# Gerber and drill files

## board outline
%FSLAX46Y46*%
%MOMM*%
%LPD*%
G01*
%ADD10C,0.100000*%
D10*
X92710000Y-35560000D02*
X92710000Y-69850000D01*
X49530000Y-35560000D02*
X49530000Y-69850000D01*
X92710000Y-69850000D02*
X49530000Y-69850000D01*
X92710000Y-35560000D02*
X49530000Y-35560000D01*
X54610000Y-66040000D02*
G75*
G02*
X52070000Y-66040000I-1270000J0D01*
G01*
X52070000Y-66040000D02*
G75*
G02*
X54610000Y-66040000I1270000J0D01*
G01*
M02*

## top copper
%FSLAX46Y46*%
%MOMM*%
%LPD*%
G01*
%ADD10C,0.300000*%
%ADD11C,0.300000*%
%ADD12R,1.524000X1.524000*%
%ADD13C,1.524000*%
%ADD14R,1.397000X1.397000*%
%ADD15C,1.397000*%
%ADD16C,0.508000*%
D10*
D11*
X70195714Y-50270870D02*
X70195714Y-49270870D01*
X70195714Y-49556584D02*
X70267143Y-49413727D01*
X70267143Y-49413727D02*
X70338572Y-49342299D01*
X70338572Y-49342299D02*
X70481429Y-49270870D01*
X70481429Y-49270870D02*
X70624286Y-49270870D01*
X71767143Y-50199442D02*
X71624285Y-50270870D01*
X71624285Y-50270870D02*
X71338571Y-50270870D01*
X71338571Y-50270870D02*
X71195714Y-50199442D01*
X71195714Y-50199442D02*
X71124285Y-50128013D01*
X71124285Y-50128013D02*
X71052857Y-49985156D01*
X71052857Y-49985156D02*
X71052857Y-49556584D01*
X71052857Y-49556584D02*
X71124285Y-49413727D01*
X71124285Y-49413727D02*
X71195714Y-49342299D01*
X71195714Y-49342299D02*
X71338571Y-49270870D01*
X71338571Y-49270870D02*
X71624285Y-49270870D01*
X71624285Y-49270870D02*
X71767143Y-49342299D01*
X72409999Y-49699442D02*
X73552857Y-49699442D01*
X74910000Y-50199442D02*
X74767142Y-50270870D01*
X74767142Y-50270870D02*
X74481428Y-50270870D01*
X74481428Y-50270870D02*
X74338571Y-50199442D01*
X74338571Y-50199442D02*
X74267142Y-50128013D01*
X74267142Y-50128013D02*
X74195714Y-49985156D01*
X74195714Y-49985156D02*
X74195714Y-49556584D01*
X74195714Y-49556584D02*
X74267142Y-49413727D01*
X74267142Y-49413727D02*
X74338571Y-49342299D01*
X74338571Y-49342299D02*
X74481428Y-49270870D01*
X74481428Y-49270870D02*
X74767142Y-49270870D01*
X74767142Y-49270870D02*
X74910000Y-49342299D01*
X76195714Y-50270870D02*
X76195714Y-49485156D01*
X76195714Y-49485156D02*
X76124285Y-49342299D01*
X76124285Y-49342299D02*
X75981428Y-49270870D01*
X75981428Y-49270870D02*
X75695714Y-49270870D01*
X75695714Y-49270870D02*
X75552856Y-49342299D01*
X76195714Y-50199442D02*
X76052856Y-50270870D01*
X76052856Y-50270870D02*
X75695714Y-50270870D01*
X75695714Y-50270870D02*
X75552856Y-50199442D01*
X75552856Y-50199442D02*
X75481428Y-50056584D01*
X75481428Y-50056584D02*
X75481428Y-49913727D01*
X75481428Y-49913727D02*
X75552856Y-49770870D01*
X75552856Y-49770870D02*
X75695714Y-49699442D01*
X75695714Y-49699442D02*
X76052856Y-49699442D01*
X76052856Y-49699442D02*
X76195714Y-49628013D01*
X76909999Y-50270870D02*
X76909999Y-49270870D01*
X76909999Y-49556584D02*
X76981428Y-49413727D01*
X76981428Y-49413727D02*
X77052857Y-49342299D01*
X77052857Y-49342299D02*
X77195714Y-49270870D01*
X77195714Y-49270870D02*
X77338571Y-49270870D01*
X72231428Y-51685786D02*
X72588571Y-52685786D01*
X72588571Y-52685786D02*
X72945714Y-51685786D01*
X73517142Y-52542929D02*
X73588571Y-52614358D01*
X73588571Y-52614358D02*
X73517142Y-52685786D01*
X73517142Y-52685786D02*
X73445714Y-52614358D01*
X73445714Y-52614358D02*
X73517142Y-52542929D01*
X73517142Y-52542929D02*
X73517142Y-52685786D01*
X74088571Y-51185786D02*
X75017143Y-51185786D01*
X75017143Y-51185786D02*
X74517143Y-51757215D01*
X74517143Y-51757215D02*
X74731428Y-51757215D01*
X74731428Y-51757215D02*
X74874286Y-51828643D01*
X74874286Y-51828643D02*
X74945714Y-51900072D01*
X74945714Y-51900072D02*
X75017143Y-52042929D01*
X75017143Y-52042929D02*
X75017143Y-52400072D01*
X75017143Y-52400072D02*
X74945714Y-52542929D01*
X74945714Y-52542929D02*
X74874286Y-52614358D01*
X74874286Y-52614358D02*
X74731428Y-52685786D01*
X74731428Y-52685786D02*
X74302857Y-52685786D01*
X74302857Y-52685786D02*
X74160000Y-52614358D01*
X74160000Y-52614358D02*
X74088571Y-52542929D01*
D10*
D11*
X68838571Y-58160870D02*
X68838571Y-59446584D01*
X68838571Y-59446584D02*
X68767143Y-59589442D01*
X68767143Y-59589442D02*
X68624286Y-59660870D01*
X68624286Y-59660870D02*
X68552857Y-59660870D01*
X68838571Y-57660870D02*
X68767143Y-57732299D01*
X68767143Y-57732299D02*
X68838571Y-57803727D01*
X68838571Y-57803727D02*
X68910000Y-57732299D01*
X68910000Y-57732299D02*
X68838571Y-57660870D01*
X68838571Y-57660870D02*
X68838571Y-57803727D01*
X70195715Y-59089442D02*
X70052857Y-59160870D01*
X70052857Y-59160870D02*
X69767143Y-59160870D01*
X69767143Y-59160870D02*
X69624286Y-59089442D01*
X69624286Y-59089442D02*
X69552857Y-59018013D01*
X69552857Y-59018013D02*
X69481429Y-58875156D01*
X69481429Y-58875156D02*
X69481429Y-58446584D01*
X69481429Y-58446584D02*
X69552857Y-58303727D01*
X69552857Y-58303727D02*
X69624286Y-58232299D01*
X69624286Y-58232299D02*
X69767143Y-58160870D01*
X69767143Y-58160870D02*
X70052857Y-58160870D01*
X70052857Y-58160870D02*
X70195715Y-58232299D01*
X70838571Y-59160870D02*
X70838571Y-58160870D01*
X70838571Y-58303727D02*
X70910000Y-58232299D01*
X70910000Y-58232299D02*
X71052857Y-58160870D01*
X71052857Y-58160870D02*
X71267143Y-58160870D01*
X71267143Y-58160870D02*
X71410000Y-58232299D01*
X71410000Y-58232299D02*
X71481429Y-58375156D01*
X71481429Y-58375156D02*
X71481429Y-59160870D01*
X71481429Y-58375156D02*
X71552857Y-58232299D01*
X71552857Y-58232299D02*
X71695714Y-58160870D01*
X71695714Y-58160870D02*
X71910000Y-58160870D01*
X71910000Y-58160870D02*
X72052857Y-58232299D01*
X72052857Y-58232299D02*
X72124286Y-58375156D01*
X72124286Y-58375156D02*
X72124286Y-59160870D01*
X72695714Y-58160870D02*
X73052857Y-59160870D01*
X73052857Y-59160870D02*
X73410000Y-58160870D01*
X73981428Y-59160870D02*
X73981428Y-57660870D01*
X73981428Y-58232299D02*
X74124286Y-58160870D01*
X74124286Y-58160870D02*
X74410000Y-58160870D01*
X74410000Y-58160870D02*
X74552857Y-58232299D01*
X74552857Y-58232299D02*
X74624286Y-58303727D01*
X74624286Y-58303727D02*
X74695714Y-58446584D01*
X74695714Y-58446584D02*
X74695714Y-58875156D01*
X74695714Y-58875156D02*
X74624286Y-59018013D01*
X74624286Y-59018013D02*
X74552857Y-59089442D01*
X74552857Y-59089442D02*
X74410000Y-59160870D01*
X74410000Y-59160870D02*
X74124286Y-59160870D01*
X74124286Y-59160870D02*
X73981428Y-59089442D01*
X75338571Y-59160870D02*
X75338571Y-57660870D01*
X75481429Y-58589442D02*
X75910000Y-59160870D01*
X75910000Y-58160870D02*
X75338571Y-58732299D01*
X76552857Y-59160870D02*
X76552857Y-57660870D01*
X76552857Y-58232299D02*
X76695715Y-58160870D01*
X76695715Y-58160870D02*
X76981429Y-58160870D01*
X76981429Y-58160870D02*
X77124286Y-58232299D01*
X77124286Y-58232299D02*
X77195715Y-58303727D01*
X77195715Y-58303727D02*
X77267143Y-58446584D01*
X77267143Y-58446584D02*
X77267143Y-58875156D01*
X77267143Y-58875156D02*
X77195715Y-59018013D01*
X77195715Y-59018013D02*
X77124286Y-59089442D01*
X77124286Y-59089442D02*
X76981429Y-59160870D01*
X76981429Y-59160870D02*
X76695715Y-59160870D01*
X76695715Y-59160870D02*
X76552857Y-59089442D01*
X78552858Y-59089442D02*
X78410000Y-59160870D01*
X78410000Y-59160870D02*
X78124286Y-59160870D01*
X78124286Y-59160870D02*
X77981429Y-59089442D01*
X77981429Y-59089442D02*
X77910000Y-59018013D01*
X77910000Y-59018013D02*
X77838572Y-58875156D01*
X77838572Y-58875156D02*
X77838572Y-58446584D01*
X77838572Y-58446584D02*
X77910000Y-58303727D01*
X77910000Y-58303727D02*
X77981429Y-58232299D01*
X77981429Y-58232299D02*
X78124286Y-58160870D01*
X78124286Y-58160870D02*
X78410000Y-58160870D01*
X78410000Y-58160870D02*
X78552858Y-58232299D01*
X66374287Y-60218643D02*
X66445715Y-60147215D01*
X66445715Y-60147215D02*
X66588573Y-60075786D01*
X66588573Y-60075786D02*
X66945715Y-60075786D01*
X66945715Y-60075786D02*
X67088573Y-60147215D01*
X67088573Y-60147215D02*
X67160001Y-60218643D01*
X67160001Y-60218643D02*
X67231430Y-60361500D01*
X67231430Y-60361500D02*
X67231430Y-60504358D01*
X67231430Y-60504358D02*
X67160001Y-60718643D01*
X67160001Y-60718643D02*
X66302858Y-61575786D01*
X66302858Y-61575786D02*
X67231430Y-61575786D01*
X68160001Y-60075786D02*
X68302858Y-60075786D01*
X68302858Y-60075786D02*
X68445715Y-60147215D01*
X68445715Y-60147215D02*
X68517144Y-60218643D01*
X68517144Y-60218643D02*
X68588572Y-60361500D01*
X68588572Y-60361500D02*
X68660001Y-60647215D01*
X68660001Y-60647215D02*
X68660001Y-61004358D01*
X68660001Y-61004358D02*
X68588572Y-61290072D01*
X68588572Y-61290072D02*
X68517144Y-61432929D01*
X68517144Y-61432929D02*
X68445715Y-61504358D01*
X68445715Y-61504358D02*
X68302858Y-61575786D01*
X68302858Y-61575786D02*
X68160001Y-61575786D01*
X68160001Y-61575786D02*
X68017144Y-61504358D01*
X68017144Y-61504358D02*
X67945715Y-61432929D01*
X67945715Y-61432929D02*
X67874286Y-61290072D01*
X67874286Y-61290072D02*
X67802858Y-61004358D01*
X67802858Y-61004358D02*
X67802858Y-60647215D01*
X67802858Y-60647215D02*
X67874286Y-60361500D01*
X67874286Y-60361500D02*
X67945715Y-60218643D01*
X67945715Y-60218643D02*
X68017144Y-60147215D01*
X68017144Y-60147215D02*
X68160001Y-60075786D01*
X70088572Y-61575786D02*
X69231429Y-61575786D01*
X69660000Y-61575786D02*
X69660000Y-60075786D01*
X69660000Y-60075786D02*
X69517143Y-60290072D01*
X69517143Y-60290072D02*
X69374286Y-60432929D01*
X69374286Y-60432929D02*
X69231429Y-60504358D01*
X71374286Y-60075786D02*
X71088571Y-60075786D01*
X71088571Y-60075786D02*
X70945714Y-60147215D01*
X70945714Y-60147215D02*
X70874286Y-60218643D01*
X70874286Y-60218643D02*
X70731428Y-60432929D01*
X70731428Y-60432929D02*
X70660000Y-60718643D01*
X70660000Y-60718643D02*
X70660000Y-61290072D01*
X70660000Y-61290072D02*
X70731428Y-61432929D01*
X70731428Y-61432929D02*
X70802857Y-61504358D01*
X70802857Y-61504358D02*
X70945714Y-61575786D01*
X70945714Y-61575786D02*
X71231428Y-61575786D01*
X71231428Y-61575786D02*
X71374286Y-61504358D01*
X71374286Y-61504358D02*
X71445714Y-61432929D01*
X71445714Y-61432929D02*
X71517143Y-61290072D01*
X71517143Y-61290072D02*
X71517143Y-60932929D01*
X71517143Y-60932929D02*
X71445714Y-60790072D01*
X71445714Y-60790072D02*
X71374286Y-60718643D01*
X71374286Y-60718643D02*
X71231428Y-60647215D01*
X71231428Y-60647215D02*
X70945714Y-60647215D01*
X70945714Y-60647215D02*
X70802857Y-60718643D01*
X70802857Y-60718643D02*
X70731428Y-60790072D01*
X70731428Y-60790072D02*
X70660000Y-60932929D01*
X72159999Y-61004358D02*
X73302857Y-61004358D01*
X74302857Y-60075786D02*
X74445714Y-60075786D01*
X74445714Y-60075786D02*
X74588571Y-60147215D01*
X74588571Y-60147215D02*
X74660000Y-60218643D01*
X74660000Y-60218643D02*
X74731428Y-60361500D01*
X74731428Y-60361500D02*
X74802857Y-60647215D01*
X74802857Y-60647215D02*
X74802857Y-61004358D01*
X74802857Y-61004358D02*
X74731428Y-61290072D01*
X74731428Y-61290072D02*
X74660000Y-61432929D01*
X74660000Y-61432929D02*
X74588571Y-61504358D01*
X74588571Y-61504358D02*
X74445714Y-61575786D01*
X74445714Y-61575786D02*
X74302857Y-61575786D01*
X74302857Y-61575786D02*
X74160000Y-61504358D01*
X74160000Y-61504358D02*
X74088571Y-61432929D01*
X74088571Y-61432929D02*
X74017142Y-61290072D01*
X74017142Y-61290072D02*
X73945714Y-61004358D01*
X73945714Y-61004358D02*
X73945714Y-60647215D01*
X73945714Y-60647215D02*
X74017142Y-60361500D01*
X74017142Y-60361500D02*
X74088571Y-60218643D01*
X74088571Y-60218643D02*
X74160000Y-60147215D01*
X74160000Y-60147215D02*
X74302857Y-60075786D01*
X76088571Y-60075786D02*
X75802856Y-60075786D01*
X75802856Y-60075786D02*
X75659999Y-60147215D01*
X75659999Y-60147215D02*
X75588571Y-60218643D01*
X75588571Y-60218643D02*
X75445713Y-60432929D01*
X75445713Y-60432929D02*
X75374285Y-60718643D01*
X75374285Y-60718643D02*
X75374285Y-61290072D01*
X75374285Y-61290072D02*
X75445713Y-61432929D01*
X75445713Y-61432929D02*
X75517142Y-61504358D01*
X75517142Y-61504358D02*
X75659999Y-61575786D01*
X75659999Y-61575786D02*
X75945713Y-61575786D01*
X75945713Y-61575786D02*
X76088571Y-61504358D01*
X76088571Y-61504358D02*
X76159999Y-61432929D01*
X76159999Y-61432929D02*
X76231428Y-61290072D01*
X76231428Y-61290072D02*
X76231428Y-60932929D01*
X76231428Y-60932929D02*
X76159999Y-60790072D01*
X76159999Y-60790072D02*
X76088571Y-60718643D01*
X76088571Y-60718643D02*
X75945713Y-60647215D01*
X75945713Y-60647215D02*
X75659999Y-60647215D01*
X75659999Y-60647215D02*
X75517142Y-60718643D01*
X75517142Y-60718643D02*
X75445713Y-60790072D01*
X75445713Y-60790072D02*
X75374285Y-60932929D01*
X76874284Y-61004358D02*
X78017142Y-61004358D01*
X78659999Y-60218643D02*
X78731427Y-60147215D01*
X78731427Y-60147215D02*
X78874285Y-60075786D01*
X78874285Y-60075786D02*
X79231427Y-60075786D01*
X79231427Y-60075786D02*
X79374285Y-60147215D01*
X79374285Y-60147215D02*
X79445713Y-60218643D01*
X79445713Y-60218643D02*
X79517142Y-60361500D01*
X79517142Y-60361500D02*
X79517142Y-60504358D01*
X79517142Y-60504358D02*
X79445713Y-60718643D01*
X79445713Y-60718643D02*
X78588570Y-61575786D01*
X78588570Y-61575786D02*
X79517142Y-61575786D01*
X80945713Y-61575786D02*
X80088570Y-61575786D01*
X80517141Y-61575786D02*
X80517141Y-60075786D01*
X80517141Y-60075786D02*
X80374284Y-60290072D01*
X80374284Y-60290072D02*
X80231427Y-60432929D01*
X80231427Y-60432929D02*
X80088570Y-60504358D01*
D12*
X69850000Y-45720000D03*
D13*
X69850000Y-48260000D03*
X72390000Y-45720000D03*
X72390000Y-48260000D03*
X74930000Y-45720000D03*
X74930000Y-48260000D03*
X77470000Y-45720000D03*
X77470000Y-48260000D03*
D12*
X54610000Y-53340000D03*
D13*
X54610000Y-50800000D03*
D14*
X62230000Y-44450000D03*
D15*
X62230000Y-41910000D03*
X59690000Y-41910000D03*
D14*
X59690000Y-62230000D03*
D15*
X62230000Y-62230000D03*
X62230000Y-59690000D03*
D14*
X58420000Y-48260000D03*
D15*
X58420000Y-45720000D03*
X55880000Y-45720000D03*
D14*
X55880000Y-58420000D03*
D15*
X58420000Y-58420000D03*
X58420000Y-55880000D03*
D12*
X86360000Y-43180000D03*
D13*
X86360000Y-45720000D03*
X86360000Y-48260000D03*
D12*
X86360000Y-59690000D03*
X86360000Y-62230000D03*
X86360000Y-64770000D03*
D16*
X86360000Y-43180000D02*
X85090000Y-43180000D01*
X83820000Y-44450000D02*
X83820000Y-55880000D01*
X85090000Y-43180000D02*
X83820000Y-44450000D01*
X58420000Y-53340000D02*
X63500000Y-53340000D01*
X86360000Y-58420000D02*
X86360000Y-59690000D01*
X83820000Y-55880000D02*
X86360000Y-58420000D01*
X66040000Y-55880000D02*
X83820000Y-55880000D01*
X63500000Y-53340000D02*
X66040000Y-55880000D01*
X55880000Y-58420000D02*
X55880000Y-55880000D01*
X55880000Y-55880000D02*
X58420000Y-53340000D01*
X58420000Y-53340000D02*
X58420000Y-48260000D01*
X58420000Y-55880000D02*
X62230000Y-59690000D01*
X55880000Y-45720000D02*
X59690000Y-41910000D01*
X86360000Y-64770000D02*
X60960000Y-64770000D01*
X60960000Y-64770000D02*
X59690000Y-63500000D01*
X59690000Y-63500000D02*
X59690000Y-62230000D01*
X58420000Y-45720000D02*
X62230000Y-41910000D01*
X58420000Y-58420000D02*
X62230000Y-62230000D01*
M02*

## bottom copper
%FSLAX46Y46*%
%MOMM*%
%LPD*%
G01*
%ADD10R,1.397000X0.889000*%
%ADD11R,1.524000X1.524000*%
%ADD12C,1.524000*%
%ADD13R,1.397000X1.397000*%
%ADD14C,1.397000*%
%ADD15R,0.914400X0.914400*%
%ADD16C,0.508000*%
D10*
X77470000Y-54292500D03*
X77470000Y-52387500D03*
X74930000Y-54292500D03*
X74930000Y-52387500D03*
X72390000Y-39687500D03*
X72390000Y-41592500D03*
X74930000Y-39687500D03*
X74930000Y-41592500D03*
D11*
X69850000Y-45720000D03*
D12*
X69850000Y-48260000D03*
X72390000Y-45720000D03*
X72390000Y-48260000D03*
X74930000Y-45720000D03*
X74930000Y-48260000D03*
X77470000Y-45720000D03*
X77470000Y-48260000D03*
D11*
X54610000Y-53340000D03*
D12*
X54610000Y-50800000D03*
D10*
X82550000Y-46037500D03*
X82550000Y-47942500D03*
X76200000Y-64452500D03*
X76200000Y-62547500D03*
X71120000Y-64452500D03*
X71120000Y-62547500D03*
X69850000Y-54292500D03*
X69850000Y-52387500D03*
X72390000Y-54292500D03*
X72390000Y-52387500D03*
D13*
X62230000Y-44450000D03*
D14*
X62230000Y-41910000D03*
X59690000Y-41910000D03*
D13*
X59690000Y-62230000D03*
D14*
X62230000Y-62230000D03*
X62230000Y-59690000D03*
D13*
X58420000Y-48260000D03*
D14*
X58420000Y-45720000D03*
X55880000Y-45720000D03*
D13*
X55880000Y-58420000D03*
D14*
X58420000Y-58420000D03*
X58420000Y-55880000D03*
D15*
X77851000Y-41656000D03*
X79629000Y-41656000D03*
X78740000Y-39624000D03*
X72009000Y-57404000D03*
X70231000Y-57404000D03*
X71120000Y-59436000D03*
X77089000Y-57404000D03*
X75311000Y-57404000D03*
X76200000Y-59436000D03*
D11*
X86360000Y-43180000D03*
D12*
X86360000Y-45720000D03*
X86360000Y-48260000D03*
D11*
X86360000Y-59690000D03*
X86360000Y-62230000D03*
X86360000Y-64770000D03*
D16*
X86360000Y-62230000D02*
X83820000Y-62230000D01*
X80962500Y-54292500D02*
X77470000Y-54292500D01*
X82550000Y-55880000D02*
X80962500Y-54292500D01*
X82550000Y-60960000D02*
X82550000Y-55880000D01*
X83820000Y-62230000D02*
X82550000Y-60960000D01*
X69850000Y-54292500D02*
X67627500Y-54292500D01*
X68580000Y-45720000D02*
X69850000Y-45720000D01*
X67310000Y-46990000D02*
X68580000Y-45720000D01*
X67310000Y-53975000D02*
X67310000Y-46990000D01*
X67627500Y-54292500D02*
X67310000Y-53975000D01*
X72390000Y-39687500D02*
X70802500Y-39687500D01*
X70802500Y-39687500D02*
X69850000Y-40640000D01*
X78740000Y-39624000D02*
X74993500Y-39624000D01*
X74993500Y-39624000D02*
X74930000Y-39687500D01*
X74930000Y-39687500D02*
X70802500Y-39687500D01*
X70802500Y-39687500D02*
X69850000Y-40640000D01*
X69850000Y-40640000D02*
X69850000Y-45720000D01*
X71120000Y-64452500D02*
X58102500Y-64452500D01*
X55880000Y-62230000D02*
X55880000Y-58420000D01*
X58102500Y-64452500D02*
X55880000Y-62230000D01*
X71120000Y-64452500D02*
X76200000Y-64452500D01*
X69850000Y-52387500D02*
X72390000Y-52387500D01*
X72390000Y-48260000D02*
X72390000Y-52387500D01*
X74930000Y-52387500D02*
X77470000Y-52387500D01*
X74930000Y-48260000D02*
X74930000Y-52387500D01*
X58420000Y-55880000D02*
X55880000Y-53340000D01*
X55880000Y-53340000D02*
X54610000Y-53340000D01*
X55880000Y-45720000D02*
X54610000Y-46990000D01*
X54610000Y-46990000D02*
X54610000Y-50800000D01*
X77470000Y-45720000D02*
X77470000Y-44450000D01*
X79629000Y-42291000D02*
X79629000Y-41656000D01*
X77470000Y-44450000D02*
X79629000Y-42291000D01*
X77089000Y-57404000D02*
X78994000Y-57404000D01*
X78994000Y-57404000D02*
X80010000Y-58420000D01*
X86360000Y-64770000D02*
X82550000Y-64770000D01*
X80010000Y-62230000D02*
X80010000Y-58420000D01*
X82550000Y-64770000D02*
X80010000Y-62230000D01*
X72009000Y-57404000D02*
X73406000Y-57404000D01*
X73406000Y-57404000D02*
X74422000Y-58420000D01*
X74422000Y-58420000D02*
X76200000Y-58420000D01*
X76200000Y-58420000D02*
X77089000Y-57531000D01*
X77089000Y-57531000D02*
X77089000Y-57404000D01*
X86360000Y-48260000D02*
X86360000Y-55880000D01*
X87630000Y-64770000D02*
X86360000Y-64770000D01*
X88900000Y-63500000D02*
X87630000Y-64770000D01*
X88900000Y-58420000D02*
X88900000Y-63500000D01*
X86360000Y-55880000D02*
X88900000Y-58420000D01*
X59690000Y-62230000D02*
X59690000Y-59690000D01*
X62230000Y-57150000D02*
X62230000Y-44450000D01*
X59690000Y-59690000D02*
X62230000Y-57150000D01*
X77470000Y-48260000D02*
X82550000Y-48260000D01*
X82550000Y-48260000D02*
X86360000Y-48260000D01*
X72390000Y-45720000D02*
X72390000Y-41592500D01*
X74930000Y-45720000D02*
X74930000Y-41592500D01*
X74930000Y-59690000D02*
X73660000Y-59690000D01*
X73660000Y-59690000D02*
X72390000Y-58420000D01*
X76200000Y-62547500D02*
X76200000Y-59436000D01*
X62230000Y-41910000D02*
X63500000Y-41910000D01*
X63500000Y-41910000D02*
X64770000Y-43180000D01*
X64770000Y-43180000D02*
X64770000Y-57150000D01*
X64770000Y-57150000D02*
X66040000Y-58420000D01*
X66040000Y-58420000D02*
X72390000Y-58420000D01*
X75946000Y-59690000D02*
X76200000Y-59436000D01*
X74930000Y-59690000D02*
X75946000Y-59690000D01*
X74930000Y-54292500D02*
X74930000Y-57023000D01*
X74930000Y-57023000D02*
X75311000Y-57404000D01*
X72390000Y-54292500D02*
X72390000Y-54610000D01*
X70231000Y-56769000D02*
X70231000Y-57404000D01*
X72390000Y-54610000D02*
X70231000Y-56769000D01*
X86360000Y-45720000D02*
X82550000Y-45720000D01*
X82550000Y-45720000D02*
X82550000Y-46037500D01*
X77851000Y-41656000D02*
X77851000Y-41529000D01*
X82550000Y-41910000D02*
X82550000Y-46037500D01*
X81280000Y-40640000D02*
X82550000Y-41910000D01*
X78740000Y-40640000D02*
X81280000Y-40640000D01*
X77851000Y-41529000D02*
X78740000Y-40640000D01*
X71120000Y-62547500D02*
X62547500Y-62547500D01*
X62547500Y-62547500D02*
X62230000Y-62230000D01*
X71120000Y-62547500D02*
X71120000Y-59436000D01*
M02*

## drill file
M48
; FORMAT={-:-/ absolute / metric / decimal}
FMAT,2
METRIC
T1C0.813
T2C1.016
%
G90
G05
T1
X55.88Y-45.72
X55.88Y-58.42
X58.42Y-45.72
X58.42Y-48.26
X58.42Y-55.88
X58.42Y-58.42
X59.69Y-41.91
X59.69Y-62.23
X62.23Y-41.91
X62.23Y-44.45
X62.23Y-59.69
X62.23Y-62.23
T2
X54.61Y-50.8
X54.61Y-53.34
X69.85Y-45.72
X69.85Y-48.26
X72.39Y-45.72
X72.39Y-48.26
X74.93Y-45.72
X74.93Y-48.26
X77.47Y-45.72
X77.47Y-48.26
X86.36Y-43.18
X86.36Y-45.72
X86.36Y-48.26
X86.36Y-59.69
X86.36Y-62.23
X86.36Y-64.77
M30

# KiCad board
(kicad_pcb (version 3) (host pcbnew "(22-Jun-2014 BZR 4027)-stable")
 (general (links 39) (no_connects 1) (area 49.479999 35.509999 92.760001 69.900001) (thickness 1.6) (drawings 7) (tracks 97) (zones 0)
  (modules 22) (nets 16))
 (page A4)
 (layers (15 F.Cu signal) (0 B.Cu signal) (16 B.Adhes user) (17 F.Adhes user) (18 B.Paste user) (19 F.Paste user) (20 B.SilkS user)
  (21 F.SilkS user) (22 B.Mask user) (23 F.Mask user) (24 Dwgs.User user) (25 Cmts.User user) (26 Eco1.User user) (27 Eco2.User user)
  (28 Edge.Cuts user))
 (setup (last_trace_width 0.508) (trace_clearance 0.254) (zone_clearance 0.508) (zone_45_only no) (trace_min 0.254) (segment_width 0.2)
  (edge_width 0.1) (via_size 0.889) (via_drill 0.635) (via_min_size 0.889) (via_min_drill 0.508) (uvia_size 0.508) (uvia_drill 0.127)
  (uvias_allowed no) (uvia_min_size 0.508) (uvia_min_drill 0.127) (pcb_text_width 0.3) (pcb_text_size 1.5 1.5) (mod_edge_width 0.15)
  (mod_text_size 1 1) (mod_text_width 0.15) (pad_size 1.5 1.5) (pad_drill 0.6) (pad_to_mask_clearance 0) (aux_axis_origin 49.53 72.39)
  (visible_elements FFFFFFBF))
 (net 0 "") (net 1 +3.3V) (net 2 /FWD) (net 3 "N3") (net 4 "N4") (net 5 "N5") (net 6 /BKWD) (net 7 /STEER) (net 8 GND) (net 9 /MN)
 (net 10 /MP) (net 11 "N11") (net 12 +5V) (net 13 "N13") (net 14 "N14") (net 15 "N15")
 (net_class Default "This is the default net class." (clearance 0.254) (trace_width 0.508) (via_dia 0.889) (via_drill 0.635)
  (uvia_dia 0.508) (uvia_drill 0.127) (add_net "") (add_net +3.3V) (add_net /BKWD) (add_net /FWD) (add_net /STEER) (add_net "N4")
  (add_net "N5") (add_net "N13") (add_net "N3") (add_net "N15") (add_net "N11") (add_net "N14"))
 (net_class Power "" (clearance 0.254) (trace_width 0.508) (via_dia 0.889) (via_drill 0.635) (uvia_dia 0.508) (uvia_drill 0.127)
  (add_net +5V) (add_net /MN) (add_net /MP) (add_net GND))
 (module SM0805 (layer B.Cu) (at 77.47 53.34 90)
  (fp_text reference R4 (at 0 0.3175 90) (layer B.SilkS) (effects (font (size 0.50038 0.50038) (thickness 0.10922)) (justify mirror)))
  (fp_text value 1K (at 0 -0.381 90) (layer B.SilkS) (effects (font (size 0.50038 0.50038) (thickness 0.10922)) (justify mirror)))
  (pad 1 smd rect (at -0.9525 0 90) (size 0.889 1.397) (layers B.Cu B.Paste B.Mask) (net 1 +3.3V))
  (pad 2 smd rect (at 0.9525 0 90) (size 0.889 1.397) (layers B.Cu B.Paste B.Mask) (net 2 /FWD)))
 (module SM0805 (layer B.Cu) (at 74.93 53.34 90)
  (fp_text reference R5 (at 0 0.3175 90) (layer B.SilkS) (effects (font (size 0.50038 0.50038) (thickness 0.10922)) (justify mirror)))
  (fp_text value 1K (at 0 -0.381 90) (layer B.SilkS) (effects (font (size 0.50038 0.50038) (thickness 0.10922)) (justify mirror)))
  (pad 1 smd rect (at -0.9525 0 90) (size 0.889 1.397) (layers B.Cu B.Paste B.Mask) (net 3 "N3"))
  (pad 2 smd rect (at 0.9525 0 90) (size 0.889 1.397) (layers B.Cu B.Paste B.Mask) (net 2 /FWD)))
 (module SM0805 (layer B.Cu) (at 72.39 40.64 270)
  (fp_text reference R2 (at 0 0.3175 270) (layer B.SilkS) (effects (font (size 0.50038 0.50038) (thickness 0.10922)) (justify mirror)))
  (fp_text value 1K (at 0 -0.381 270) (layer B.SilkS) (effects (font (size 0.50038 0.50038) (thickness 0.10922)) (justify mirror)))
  (pad 1 smd rect (at -0.9525 0 270) (size 0.889 1.397) (layers B.Cu B.Paste B.Mask) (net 1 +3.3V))
  (pad 2 smd rect (at 0.9525 0 270) (size 0.889 1.397) (layers B.Cu B.Paste B.Mask) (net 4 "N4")))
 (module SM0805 (layer B.Cu) (at 74.93 40.64 270)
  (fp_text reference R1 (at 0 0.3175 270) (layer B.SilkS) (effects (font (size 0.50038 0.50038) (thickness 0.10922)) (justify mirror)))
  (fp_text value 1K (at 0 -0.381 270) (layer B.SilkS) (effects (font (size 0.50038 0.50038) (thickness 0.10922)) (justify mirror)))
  (pad 1 smd rect (at -0.9525 0 270) (size 0.889 1.397) (layers B.Cu B.Paste B.Mask) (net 1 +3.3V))
  (pad 2 smd rect (at 0.9525 0 270) (size 0.889 1.397) (layers B.Cu B.Paste B.Mask) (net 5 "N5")))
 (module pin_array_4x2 (layer B.Cu) (at 73.66 46.99)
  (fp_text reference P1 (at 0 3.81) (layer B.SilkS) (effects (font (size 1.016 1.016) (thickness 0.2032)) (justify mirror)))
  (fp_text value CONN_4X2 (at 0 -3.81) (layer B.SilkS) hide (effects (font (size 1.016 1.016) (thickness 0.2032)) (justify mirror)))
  (pad 1 thru_hole rect (at -3.81 -1.27) (size 1.524 1.524) (drill 1.016) (layers *.Cu *.Mask B.SilkS) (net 1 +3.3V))
  (pad 2 thru_hole circle (at -3.81 1.27) (size 1.524 1.524) (drill 1.016) (layers *.Cu *.Mask B.SilkS))
  (pad 3 thru_hole circle (at -1.27 -1.27) (size 1.524 1.524) (drill 1.016) (layers *.Cu *.Mask B.SilkS) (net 4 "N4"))
  (pad 4 thru_hole circle (at -1.27 1.27) (size 1.524 1.524) (drill 1.016) (layers *.Cu *.Mask B.SilkS) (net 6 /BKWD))
  (pad 5 thru_hole circle (at 1.27 -1.27) (size 1.524 1.524) (drill 1.016) (layers *.Cu *.Mask B.SilkS) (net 5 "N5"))
  (pad 6 thru_hole circle (at 1.27 1.27) (size 1.524 1.524) (drill 1.016) (layers *.Cu *.Mask B.SilkS) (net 2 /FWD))
  (pad 7 thru_hole circle (at 3.81 -1.27) (size 1.524 1.524) (drill 1.016) (layers *.Cu *.Mask B.SilkS) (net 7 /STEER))
  (pad 8 thru_hole circle (at 3.81 1.27) (size 1.524 1.524) (drill 1.016) (layers *.Cu *.Mask B.SilkS) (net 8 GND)))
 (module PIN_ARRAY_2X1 (layer F.Cu) (at 54.61 52.07 90)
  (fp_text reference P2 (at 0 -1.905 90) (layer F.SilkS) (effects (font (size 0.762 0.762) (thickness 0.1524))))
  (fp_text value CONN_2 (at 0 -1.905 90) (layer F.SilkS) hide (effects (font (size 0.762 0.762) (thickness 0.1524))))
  (pad 1 thru_hole rect (at -1.27 0 90) (size 1.524 1.524) (drill 1.016) (layers *.Cu *.Mask F.SilkS) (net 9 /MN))
  (pad 2 thru_hole circle (at 1.27 0 90) (size 1.524 1.524) (drill 1.016) (layers *.Cu *.Mask F.SilkS) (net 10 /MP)))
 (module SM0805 (layer B.Cu) (at 82.55 46.99 270)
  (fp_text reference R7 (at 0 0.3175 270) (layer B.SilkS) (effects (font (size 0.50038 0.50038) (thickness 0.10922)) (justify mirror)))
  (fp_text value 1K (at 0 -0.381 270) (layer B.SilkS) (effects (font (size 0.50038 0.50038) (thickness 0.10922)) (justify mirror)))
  (pad 1 smd rect (at -0.9525 0 270) (size 0.889 1.397) (layers B.Cu B.Paste B.Mask) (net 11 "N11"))
  (pad 2 smd rect (at 0.9525 0 270) (size 0.889 1.397) (layers B.Cu B.Paste B.Mask) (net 8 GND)))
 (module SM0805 (layer B.Cu) (at 76.2 63.5 90)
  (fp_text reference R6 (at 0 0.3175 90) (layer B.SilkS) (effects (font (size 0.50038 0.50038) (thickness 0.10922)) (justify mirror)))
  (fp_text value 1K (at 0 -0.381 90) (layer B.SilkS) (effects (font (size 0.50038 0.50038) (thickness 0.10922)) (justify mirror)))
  (pad 1 smd rect (at -0.9525 0 90) (size 0.889 1.397) (layers B.Cu B.Paste B.Mask) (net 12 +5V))
  (pad 2 smd rect (at 0.9525 0 90) (size 0.889 1.397) (layers B.Cu B.Paste B.Mask) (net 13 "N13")))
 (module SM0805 (layer B.Cu) (at 71.12 63.5 90)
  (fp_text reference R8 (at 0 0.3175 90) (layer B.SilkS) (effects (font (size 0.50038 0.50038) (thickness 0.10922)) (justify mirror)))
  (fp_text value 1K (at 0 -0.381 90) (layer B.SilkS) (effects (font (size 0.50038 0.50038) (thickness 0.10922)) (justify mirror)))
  (pad 1 smd rect (at -0.9525 0 90) (size 0.889 1.397) (layers B.Cu B.Paste B.Mask) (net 12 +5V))
  (pad 2 smd rect (at 0.9525 0 90) (size 0.889 1.397) (layers B.Cu B.Paste B.Mask) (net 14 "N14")))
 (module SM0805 (layer B.Cu) (at 69.85 53.34 90)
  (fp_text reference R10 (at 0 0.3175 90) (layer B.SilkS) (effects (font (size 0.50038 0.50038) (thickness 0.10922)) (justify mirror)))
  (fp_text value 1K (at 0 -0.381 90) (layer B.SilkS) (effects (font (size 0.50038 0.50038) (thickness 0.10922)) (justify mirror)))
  (pad 1 smd rect (at -0.9525 0 90) (size 0.889 1.397) (layers B.Cu B.Paste B.Mask) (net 1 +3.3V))
  (pad 2 smd rect (at 0.9525 0 90) (size 0.889 1.397) (layers B.Cu B.Paste B.Mask) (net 6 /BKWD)))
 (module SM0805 (layer B.Cu) (at 72.39 53.34 90)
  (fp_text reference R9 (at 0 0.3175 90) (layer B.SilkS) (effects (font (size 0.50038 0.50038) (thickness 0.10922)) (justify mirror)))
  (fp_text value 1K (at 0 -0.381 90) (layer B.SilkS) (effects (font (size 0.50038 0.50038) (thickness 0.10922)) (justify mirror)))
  (pad 1 smd rect (at -0.9525 0 90) (size 0.889 1.397) (layers B.Cu B.Paste B.Mask) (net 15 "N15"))
  (pad 2 smd rect (at 0.9525 0 90) (size 0.889 1.397) (layers B.Cu B.Paste B.Mask) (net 6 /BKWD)))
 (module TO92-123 (layer F.Cu) (at 60.96 43.18 270)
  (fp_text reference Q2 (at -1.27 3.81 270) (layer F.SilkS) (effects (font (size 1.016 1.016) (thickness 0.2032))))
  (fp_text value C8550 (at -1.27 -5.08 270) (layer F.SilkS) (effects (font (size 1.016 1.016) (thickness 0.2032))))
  (pad 3 thru_hole rect (at 1.27 -1.27 270) (size 1.397 1.397) (drill 0.8128) (layers *.Cu *.Mask F.SilkS) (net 8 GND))
  (pad 2 thru_hole circle (at -1.27 -1.27 270) (size 1.397 1.397) (drill 0.8128) (layers *.Cu *.Mask F.SilkS) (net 13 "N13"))
  (pad 1 thru_hole circle (at -1.27 1.27 270) (size 1.397 1.397) (drill 0.8128) (layers *.Cu *.Mask F.SilkS) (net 10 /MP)))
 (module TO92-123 (layer F.Cu) (at 60.96 60.96 180)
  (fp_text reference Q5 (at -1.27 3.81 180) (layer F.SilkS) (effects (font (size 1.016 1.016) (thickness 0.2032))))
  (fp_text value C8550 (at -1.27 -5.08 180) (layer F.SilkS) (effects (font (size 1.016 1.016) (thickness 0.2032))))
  (pad 3 thru_hole rect (at 1.27 -1.27 180) (size 1.397 1.397) (drill 0.8128) (layers *.Cu *.Mask F.SilkS) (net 8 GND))
  (pad 2 thru_hole circle (at -1.27 -1.27 180) (size 1.397 1.397) (drill 0.8128) (layers *.Cu *.Mask F.SilkS) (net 14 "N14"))
  (pad 1 thru_hole circle (at -1.27 1.27 180) (size 1.397 1.397) (drill 0.8128) (layers *.Cu *.Mask F.SilkS) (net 9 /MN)))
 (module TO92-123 (layer F.Cu) (at 57.15 46.99 270)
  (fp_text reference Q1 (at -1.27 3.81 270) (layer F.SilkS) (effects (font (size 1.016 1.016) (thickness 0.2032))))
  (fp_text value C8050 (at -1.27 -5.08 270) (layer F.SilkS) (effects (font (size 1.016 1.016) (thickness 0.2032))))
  (pad 3 thru_hole rect (at 1.27 -1.27 270) (size 1.397 1.397) (drill 0.8128) (layers *.Cu *.Mask F.SilkS) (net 12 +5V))
  (pad 2 thru_hole circle (at -1.27 -1.27 270) (size 1.397 1.397) (drill 0.8128) (layers *.Cu *.Mask F.SilkS) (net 13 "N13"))
  (pad 1 thru_hole circle (at -1.27 1.27 270) (size 1.397 1.397) (drill 0.8128) (layers *.Cu *.Mask F.SilkS) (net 10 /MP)))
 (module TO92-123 (layer F.Cu) (at 57.15 57.15 180)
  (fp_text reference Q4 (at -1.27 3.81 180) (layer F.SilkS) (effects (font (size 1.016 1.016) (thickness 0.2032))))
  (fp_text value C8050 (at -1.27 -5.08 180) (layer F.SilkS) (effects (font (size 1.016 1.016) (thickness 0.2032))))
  (pad 3 thru_hole rect (at 1.27 -1.27 180) (size 1.397 1.397) (drill 0.8128) (layers *.Cu *.Mask F.SilkS) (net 12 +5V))
  (pad 2 thru_hole circle (at -1.27 -1.27 180) (size 1.397 1.397) (drill 0.8128) (layers *.Cu *.Mask F.SilkS) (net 14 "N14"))
  (pad 1 thru_hole circle (at -1.27 1.27 180) (size 1.397 1.397) (drill 0.8128) (layers *.Cu *.Mask F.SilkS) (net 9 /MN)))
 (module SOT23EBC (layer B.Cu) (at 78.74 40.64)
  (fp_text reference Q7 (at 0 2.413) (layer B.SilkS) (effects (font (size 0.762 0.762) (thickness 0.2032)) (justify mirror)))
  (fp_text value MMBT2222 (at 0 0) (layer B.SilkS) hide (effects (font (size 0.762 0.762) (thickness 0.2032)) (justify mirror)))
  (pad 1 smd rect (at -0.889 1.016) (size 0.9144 0.9144) (layers B.Cu B.Paste B.Mask) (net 11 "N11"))
  (pad 2 smd rect (at 0.889 1.016) (size 0.9144 0.9144) (layers B.Cu B.Paste B.Mask) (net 7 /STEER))
  (pad 3 smd rect (at 0 -1.016) (size 0.9144 0.9144) (layers B.Cu B.Paste B.Mask) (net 1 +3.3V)))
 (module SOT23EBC (layer B.Cu) (at 71.12 58.42 180)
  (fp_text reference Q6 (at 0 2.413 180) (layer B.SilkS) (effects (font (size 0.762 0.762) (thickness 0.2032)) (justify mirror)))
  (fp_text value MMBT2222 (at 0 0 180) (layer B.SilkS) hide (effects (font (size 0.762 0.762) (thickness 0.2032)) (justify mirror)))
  (pad 1 smd rect (at -0.889 1.016 180) (size 0.9144 0.9144) (layers B.Cu B.Paste B.Mask) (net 8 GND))
  (pad 2 smd rect (at 0.889 1.016 180) (size 0.9144 0.9144) (layers B.Cu B.Paste B.Mask) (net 15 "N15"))
  (pad 3 smd rect (at 0 -1.016 180) (size 0.9144 0.9144) (layers B.Cu B.Paste B.Mask) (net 14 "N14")))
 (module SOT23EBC (layer B.Cu) (at 76.2 58.42 180)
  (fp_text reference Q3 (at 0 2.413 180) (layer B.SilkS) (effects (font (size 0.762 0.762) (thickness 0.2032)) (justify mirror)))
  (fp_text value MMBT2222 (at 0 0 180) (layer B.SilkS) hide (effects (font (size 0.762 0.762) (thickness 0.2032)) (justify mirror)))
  (pad 1 smd rect (at -0.889 1.016 180) (size 0.9144 0.9144) (layers B.Cu B.Paste B.Mask) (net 8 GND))
  (pad 2 smd rect (at 0.889 1.016 180) (size 0.9144 0.9144) (layers B.Cu B.Paste B.Mask) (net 3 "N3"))
  (pad 3 smd rect (at 0 -1.016 180) (size 0.9144 0.9144) (layers B.Cu B.Paste B.Mask) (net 13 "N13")))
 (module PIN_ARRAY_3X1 (layer F.Cu) (at 86.36 45.72 270)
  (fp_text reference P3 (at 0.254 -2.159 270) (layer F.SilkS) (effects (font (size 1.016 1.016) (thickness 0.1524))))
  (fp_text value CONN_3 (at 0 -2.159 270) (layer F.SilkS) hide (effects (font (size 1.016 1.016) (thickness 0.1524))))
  (pad 1 thru_hole rect (at -2.54 0 270) (size 1.524 1.524) (drill 1.016) (layers *.Cu *.Mask F.SilkS) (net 12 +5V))
  (pad 2 thru_hole circle (at 0 0 270) (size 1.524 1.524) (drill 1.016) (layers *.Cu *.Mask F.SilkS) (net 11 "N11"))
  (pad 3 thru_hole circle (at 2.54 0 270) (size 1.524 1.524) (drill 1.016) (layers *.Cu *.Mask F.SilkS) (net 8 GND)))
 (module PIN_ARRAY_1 (layer F.Cu) (at 86.36 59.69)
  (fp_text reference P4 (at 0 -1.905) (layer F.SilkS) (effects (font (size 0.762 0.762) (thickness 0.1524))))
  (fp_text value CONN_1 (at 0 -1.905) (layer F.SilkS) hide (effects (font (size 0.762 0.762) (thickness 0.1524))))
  (pad 1 thru_hole rect (at 0 0) (size 1.524 1.524) (drill 1.016) (layers *.Cu *.Mask F.SilkS) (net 12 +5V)))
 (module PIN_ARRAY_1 (layer F.Cu) (at 86.36 62.23)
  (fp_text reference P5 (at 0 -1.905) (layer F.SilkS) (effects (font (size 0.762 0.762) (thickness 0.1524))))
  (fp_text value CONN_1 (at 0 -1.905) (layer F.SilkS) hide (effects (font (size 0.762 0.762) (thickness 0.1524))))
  (pad 1 thru_hole rect (at 0 0) (size 1.524 1.524) (drill 1.016) (layers *.Cu *.Mask F.SilkS) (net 1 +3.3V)))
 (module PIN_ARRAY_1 (layer F.Cu) (at 86.36 64.77)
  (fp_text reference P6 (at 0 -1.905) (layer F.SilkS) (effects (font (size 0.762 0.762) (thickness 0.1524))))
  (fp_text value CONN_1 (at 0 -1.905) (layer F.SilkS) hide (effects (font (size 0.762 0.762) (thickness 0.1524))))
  (pad 1 thru_hole rect (at 0 0) (size 1.524 1.524) (drill 1.016) (layers *.Cu *.Mask F.SilkS) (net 8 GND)))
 (gr_line (start 92.71 35.56) (end 92.71 69.85) (angle 90) (layer Edge.Cuts) (width 0.1))
 (gr_line (start 49.53 35.56) (end 49.53 69.85) (angle 90) (layer Edge.Cuts) (width 0.1))
 (gr_line (start 92.71 69.85) (end 49.53 69.85) (angle 90) (layer Edge.Cuts) (width 0.1))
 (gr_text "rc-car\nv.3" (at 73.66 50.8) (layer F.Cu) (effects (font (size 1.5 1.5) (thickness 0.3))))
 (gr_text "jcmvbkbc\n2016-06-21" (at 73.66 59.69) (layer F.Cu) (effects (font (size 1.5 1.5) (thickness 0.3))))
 (gr_line (start 92.71 35.56) (end 49.53 35.56) (angle 90) (layer Edge.Cuts) (width 0.1))
 (gr_circle (center 53.34 66.04) (end 54.61 66.04) (layer Edge.Cuts) (width 0.1))
 (segment (start 86.36 62.23) (end 83.82 62.23) (width 0.508) (layer B.Cu) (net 1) (status 400000))
 (segment (start 80.9625 54.2925) (end 77.47 54.2925) (width 0.508) (layer B.Cu) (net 1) (status 800000))
 (segment (start 82.55 55.88) (end 80.9625 54.2925) (width 0.508) (layer B.Cu) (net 1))
 (segment (start 82.55 60.96) (end 82.55 55.88) (width 0.508) (layer B.Cu) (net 1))
 (segment (start 83.82 62.23) (end 82.55 60.96) (width 0.508) (layer B.Cu) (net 1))
 (segment (start 69.85 54.2925) (end 67.6275 54.2925) (width 0.508) (layer B.Cu) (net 1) (status 400000))
 (segment (start 68.58 45.72) (end 69.85 45.72) (width 0.508) (layer B.Cu) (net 1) (status 800000))
 (segment (start 67.31 46.99) (end 68.58 45.72) (width 0.508) (layer B.Cu) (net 1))
 (segment (start 67.31 53.975) (end 67.31 46.99) (width 0.508) (layer B.Cu) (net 1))
 (segment (start 67.6275 54.2925) (end 67.31 53.975) (width 0.508) (layer B.Cu) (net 1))
 (segment (start 72.39 39.6875) (end 70.8025 39.6875) (width 0.508) (layer B.Cu) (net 1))
 (segment (start 70.8025 39.6875) (end 69.85 40.64) (width 0.508) (layer B.Cu) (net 1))
 (segment (start 78.74 39.624) (end 74.9935 39.624) (width 0.508) (layer B.Cu) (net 1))
 (segment (start 74.9935 39.624) (end 74.93 39.6875) (width 0.508) (layer B.Cu) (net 1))
 (segment (start 74.93 39.6875) (end 70.8025 39.6875) (width 0.508) (layer B.Cu) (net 1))
 (segment (start 70.8025 39.6875) (end 69.85 40.64) (width 0.508) (layer B.Cu) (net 1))
 (segment (start 69.85 40.64) (end 69.85 45.72) (width 0.508) (layer B.Cu) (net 1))
 (segment (start 71.12 64.4525) (end 58.1025 64.4525) (width 0.508) (layer B.Cu) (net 12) (status 400000))
 (segment (start 55.88 62.23) (end 55.88 58.42) (width 0.508) (layer B.Cu) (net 12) (status 800000))
 (segment (start 58.1025 64.4525) (end 55.88 62.23) (width 0.508) (layer B.Cu) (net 12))
 (segment (start 71.12 64.4525) (end 76.2 64.4525) (width 0.508) (layer B.Cu) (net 12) (status C00000))
 (segment (start 86.36 43.18) (end 85.09 43.18) (width 0.508) (layer F.Cu) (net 12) (status 400000))
 (segment (start 83.82 44.45) (end 83.82 55.88) (width 0.508) (layer F.Cu) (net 12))
 (segment (start 85.09 43.18) (end 83.82 44.45) (width 0.508) (layer F.Cu) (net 12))
 (segment (start 58.42 53.34) (end 63.5 53.34) (width 0.508) (layer F.Cu) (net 12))
 (segment (start 86.36 58.42) (end 86.36 59.69) (width 0.508) (layer F.Cu) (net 12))
 (segment (start 83.82 55.88) (end 86.36 58.42) (width 0.508) (layer F.Cu) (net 12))
 (segment (start 66.04 55.88) (end 83.82 55.88) (width 0.508) (layer F.Cu) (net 12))
 (segment (start 63.5 53.34) (end 66.04 55.88) (width 0.508) (layer F.Cu) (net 12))
 (segment (start 55.88 58.42) (end 55.88 55.88) (width 0.508) (layer F.Cu) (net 12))
 (segment (start 55.88 55.88) (end 58.42 53.34) (width 0.508) (layer F.Cu) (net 12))
 (segment (start 58.42 53.34) (end 58.42 48.26) (width 0.508) (layer F.Cu) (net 12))
 (segment (start 69.85 52.3875) (end 72.39 52.3875) (width 0.508) (layer B.Cu) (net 6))
 (segment (start 72.39 48.26) (end 72.39 52.3875) (width 0.508) (layer B.Cu) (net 6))
 (segment (start 74.93 52.3875) (end 77.47 52.3875) (width 0.508) (layer B.Cu) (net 2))
 (segment (start 74.93 48.26) (end 74.93 52.3875) (width 0.508) (layer B.Cu) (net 2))
 (segment (start 58.42 55.88) (end 55.88 53.34) (width 0.508) (layer B.Cu) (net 9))
 (segment (start 55.88 53.34) (end 54.61 53.34) (width 0.508) (layer B.Cu) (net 9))
 (segment (start 58.42 55.88) (end 62.23 59.69) (width 0.508) (layer F.Cu) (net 9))
 (segment (start 55.88 45.72) (end 54.61 46.99) (width 0.508) (layer B.Cu) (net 10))
 (segment (start 54.61 46.99) (end 54.61 50.8) (width 0.508) (layer B.Cu) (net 10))
 (segment (start 55.88 45.72) (end 59.69 41.91) (width 0.508) (layer F.Cu) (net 10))
 (segment (start 77.47 45.72) (end 77.47 44.45) (width 0.508) (layer B.Cu) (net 7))
 (segment (start 79.629 42.291) (end 79.629 41.656) (width 0.508) (layer B.Cu) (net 7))
 (segment (start 77.47 44.45) (end 79.629 42.291) (width 0.508) (layer B.Cu) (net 7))
 (segment (start 77.089 57.404) (end 78.994 57.404) (width 0.508) (layer B.Cu) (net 8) (status 400000))
 (segment (start 78.994 57.404) (end 80.01 58.42) (width 0.508) (layer B.Cu) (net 8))
 (segment (start 86.36 64.77) (end 82.55 64.77) (width 0.508) (layer B.Cu) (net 8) (status 400000))
 (segment (start 80.01 62.23) (end 80.01 58.42) (width 0.508) (layer B.Cu) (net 8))
 (segment (start 82.55 64.77) (end 80.01 62.23) (width 0.508) (layer B.Cu) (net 8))
 (segment (start 72.009 57.404) (end 73.406 57.404) (width 0.508) (layer B.Cu) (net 8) (status 400000))
 (segment (start 73.406 57.404) (end 74.422 58.42) (width 0.508) (layer B.Cu) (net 8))
 (segment (start 74.422 58.42) (end 76.2 58.42) (width 0.508) (layer B.Cu) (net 8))
 (segment (start 76.2 58.42) (end 77.089 57.531) (width 0.508) (layer B.Cu) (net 8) (status 800000))
 (segment (start 77.089 57.531) (end 77.089 57.404) (width 0.508) (layer B.Cu) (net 8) (status C00000))
 (segment (start 86.36 48.26) (end 86.36 55.88) (width 0.508) (layer B.Cu) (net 8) (status 400000))
 (segment (start 87.63 64.77) (end 86.36 64.77) (width 0.508) (layer B.Cu) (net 8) (status 800000))
 (segment (start 88.9 63.5) (end 87.63 64.77) (width 0.508) (layer B.Cu) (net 8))
 (segment (start 88.9 58.42) (end 88.9 63.5) (width 0.508) (layer B.Cu) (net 8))
 (segment (start 86.36 55.88) (end 88.9 58.42) (width 0.508) (layer B.Cu) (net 8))
 (segment (start 59.69 62.23) (end 59.69 59.69) (width 0.508) (layer B.Cu) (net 8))
 (segment (start 62.23 57.15) (end 62.23 44.45) (width 0.508) (layer B.Cu) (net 8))
 (segment (start 59.69 59.69) (end 62.23 57.15) (width 0.508) (layer B.Cu) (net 8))
 (segment (start 86.36 64.77) (end 60.96 64.77) (width 0.508) (layer F.Cu) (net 8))
 (segment (start 60.96 64.77) (end 59.69 63.5) (width 0.508) (layer F.Cu) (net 8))
 (segment (start 59.69 63.5) (end 59.69 62.23) (width 0.508) (layer F.Cu) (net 8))
 (segment (start 77.47 48.26) (end 82.55 48.26) (width 0.508) (layer B.Cu) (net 8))
 (segment (start 82.55 48.26) (end 86.36 48.26) (width 0.508) (layer B.Cu) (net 8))
 (segment (start 72.39 45.72) (end 72.39 41.5925) (width 0.508) (layer B.Cu) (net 4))
 (segment (start 74.93 45.72) (end 74.93 41.5925) (width 0.508) (layer B.Cu) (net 5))
 (segment (start 74.93 59.69) (end 73.66 59.69) (width 0.508) (layer B.Cu) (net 13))
 (segment (start 73.66 59.69) (end 72.39 58.42) (width 0.508) (layer B.Cu) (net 13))
 (segment (start 76.2 62.5475) (end 76.2 59.436) (width 0.508) (layer B.Cu) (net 13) (status C00000))
 (segment (start 62.23 41.91) (end 63.5 41.91) (width 0.508) (layer B.Cu) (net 13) (status 400000))
 (segment (start 63.5 41.91) (end 64.77 43.18) (width 0.508) (layer B.Cu) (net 13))
 (segment (start 64.77 43.18) (end 64.77 57.15) (width 0.508) (layer B.Cu) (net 13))
 (segment (start 64.77 57.15) (end 66.04 58.42) (width 0.508) (layer B.Cu) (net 13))
 (segment (start 66.04 58.42) (end 72.39 58.42) (width 0.508) (layer B.Cu) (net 13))
 (segment (start 75.946 59.69) (end 76.2 59.436) (width 0.508) (layer B.Cu) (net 13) (status C00000))
 (segment (start 74.93 59.69) (end 75.946 59.69) (width 0.508) (layer B.Cu) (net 13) (status 800000))
 (segment (start 58.42 45.72) (end 62.23 41.91) (width 0.508) (layer F.Cu) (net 13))
 (segment (start 74.93 54.2925) (end 74.93 57.023) (width 0.508) (layer B.Cu) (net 3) (status C00000))
 (segment (start 74.93 57.023) (end 75.311 57.404) (width 0.508) (layer B.Cu) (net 3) (status C00000))
 (segment (start 72.39 54.2925) (end 72.39 54.61) (width 0.508) (layer B.Cu) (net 15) (status C00000))
 (segment (start 70.231 56.769) (end 70.231 57.404) (width 0.508) (layer B.Cu) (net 15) (status 800000))
 (segment (start 72.39 54.61) (end 70.231 56.769) (width 0.508) (layer B.Cu) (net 15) (status 400000))
 (segment (start 86.36 45.72) (end 82.55 45.72) (width 0.508) (layer B.Cu) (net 11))
 (segment (start 82.55 45.72) (end 82.55 46.0375) (width 0.508) (layer B.Cu) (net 11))
 (segment (start 77.851 41.656) (end 77.851 41.529) (width 0.508) (layer B.Cu) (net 11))
 (segment (start 82.55 41.91) (end 82.55 46.0375) (width 0.508) (layer B.Cu) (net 11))
 (segment (start 81.28 40.64) (end 82.55 41.91) (width 0.508) (layer B.Cu) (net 11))
 (segment (start 78.74 40.64) (end 81.28 40.64) (width 0.508) (layer B.Cu) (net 11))
 (segment (start 77.851 41.529) (end 78.74 40.64) (width 0.508) (layer B.Cu) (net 11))
 (segment (start 71.12 62.5475) (end 62.5475 62.5475) (width 0.508) (layer B.Cu) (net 14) (status C00000))
 (segment (start 62.5475 62.5475) (end 62.23 62.23) (width 0.508) (layer B.Cu) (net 14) (status C00000))
 (segment (start 71.12 62.5475) (end 71.12 59.436) (width 0.508) (layer B.Cu) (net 14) (status C00000))
 (segment (start 58.42 58.42) (end 62.23 62.23) (width 0.508) (layer F.Cu) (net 14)))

